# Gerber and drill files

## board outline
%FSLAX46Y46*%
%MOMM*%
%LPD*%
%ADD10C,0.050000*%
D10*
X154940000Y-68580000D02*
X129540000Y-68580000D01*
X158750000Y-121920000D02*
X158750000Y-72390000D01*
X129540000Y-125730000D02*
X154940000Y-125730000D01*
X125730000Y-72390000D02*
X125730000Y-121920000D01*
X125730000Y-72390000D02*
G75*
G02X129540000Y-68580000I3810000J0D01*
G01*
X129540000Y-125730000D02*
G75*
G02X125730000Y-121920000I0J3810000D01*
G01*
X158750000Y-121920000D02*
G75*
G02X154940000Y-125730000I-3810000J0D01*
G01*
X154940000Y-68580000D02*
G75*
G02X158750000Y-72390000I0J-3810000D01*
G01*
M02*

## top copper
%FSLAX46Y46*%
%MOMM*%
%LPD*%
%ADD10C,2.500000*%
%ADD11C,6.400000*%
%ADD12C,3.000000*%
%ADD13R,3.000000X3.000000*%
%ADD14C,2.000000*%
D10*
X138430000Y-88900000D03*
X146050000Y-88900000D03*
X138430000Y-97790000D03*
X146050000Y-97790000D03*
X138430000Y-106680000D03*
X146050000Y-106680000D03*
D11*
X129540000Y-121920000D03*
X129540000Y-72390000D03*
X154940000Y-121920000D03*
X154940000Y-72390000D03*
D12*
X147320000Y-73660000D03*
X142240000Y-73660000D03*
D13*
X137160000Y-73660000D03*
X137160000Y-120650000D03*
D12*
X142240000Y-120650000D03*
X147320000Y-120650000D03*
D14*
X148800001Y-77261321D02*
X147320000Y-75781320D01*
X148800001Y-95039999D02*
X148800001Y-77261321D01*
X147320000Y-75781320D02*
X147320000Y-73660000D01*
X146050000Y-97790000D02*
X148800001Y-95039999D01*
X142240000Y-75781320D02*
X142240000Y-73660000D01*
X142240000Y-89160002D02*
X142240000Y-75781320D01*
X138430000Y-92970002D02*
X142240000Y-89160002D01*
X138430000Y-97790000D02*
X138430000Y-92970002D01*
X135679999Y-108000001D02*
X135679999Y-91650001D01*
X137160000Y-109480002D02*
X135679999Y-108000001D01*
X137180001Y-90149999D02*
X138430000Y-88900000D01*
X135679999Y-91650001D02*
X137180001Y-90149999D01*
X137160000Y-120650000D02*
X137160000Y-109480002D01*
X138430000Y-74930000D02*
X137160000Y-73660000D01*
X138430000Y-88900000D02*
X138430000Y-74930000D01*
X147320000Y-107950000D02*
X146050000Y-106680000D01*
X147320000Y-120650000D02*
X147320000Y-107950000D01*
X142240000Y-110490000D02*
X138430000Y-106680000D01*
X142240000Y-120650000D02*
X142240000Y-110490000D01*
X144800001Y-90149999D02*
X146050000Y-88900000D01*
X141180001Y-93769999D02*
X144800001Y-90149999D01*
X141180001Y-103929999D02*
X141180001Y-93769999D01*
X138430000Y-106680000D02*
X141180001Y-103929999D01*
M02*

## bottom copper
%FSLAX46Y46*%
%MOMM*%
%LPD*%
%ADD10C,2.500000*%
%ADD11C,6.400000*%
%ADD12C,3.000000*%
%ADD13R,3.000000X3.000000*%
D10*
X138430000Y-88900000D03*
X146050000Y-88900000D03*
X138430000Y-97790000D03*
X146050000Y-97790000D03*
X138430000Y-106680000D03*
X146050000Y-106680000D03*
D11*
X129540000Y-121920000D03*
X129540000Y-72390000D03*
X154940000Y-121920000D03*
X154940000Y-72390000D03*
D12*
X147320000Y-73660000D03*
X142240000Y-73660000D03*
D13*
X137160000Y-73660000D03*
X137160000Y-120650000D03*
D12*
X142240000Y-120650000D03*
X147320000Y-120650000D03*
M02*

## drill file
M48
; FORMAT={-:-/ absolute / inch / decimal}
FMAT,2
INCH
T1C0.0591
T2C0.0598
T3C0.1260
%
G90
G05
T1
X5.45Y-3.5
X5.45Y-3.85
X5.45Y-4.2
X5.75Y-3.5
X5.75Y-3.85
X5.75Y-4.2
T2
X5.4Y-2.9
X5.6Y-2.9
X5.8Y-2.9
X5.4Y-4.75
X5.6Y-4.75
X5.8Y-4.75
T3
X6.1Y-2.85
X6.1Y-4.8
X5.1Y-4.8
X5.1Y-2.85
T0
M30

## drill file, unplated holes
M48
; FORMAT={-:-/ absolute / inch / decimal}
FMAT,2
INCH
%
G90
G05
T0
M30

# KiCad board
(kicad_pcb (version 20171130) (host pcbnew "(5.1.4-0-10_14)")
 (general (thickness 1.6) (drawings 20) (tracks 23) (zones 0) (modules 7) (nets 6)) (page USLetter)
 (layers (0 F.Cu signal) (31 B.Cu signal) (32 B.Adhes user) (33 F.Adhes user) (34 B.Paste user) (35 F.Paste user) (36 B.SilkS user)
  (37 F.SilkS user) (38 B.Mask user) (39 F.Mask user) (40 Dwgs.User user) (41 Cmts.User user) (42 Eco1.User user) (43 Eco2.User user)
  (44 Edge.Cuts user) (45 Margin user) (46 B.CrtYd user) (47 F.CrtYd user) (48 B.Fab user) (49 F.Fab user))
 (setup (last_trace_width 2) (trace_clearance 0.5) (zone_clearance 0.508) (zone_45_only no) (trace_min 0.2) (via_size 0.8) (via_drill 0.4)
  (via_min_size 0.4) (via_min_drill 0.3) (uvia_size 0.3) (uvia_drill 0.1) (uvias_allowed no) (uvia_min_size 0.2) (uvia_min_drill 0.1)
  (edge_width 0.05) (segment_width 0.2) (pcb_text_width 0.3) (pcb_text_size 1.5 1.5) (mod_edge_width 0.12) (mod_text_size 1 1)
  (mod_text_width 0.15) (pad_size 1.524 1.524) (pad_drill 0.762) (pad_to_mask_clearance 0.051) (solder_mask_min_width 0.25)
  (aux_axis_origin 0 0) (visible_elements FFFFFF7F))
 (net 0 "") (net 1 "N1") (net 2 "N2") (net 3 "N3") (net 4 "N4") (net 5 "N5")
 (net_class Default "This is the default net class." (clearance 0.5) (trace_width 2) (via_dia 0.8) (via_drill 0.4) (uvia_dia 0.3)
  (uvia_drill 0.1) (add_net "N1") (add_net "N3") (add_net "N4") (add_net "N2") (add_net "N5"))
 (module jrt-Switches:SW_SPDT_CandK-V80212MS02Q (layer F.Cu) (at 142.24 97.79)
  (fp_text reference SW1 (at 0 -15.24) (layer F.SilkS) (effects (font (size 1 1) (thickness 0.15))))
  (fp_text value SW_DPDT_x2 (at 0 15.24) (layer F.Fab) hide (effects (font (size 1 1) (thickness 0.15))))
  (pad 1 thru_hole circle (at -3.81 -8.89) (size 2.5 2.5) (drill 1.5) (layers *.Cu *.Mask) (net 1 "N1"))
  (pad 4 thru_hole circle (at 3.81 -8.89) (size 2.5 2.5) (drill 1.5) (layers *.Cu *.Mask) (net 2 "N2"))
  (pad 2 thru_hole circle (at -3.81 0) (size 2.5 2.5) (drill 1.5) (layers *.Cu *.Mask) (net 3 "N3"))
  (pad 5 thru_hole circle (at 3.81 0) (size 2.5 2.5) (drill 1.5) (layers *.Cu *.Mask) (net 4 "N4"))
  (pad 3 thru_hole circle (at -3.81 8.89) (size 2.5 2.5) (drill 1.5) (layers *.Cu *.Mask) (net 2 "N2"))
  (pad 6 thru_hole circle (at 3.81 8.89) (size 2.5 2.5) (drill 1.5) (layers *.Cu *.Mask) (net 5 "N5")))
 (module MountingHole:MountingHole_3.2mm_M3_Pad (layer F.Cu) (at 129.54 121.92)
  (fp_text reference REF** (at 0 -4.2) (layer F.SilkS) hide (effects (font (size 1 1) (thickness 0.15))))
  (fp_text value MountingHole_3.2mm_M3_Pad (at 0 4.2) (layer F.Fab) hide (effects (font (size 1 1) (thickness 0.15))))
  (pad 1 thru_hole circle (at 0 0) (size 6.4 6.4) (drill 3.2) (layers *.Cu *.Mask)))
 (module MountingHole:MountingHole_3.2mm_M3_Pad (layer F.Cu) (at 129.54 72.39)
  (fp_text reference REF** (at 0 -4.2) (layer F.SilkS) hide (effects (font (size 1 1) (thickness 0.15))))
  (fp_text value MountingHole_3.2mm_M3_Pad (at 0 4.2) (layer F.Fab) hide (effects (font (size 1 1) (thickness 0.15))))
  (pad 1 thru_hole circle (at 0 0) (size 6.4 6.4) (drill 3.2) (layers *.Cu *.Mask)))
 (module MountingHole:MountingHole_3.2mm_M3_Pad (layer F.Cu) (at 154.94 121.92)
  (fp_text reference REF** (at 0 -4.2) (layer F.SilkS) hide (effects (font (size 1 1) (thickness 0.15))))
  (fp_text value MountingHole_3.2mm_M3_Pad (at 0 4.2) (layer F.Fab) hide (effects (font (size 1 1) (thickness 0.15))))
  (pad 1 thru_hole circle (at 0 0) (size 6.4 6.4) (drill 3.2) (layers *.Cu *.Mask)))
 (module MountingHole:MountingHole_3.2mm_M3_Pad (layer F.Cu) (at 154.94 72.39)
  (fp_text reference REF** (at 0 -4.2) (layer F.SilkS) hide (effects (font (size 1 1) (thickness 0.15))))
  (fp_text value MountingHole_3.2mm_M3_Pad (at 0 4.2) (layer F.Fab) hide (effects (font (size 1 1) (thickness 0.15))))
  (pad 1 thru_hole circle (at 0 0) (size 6.4 6.4) (drill 3.2) (layers *.Cu *.Mask)))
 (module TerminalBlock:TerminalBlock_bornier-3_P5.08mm (layer F.Cu) (at 137.16 73.66)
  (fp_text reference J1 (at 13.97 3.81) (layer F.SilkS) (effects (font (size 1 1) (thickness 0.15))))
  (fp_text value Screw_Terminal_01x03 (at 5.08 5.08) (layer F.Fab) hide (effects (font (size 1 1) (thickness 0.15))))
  (pad 3 thru_hole circle (at 10.16 0) (size 3 3) (drill 1.52) (layers *.Cu *.Mask) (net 4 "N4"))
  (pad 2 thru_hole circle (at 5.08 0) (size 3 3) (drill 1.52) (layers *.Cu *.Mask) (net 3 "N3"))
  (pad 1 thru_hole rect (at 0 0) (size 3 3) (drill 1.52) (layers *.Cu *.Mask) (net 1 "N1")))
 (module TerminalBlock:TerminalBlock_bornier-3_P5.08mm (layer F.Cu) (at 137.16 120.65)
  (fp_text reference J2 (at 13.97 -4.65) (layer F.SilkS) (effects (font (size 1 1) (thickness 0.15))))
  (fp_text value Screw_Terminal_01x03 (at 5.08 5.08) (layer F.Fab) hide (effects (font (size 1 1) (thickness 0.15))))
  (pad 1 thru_hole rect (at 0 0) (size 3 3) (drill 1.52) (layers *.Cu *.Mask) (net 1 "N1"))
  (pad 2 thru_hole circle (at 5.08 0) (size 3 3) (drill 1.52) (layers *.Cu *.Mask) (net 2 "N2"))
  (pad 3 thru_hole circle (at 10.16 0) (size 3 3) (drill 1.52) (layers *.Cu *.Mask) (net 5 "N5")))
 (gr_line (start 154.94 68.58) (end 129.54 68.58) (layer Edge.Cuts) (width 0.05))
 (gr_line (start 158.75 121.92) (end 158.75 72.39) (layer Edge.Cuts) (width 0.05))
 (gr_line (start 129.54 125.73) (end 154.94 125.73) (layer Edge.Cuts) (width 0.05))
 (gr_line (start 125.73 72.39) (end 125.73 121.92) (layer Edge.Cuts) (width 0.05))
 (gr_arc (start 129.54 72.39) (end 129.54 68.58) (angle -90) (layer Edge.Cuts) (width 0.05))
 (gr_arc (start 129.54 121.92) (end 125.73 121.92) (angle -90) (layer Edge.Cuts) (width 0.05))
 (gr_arc (start 154.94 121.92) (end 154.94 125.73) (angle -90) (layer Edge.Cuts) (width 0.05))
 (gr_arc (start 154.94 72.39) (end 158.75 72.39) (angle -90) (layer Edge.Cuts) (width 0.05))
 (segment (start 148.800001 77.261321) (end 147.32 75.78132) (width 2) (layer F.Cu) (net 4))
 (segment (start 148.800001 95.039999) (end 148.800001 77.261321) (width 2) (layer F.Cu) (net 4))
 (segment (start 147.32 75.78132) (end 147.32 73.66) (width 2) (layer F.Cu) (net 4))
 (segment (start 146.05 97.79) (end 148.800001 95.039999) (width 2) (layer F.Cu) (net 4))
 (segment (start 142.24 75.78132) (end 142.24 73.66) (width 2) (layer F.Cu) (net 3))
 (segment (start 142.24 89.160002) (end 142.24 75.78132) (width 2) (layer F.Cu) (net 3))
 (segment (start 138.43 92.970002) (end 142.24 89.160002) (width 2) (layer F.Cu) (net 3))
 (segment (start 138.43 97.79) (end 138.43 92.970002) (width 2) (layer F.Cu) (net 3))
 (segment (start 135.679999 108.000001) (end 135.679999 91.650001) (width 2) (layer F.Cu) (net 1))
 (segment (start 137.16 109.480002) (end 135.679999 108.000001) (width 2) (layer F.Cu) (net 1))
 (segment (start 137.180001 90.149999) (end 138.43 88.9) (width 2) (layer F.Cu) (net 1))
 (segment (start 135.679999 91.650001) (end 137.180001 90.149999) (width 2) (layer F.Cu) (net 1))
 (segment (start 137.16 120.65) (end 137.16 109.480002) (width 2) (layer F.Cu) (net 1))
 (segment (start 138.43 74.93) (end 137.16 73.66) (width 2) (layer F.Cu) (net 1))
 (segment (start 138.43 88.9) (end 138.43 74.93) (width 2) (layer F.Cu) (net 1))
 (segment (start 147.32 107.95) (end 146.05 106.68) (width 2) (layer F.Cu) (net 5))
 (segment (start 147.32 120.65) (end 147.32 107.95) (width 2) (layer F.Cu) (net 5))
 (segment (start 142.24 110.49) (end 138.43 106.68) (width 2) (layer F.Cu) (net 2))
 (segment (start 142.24 120.65) (end 142.24 110.49) (width 2) (layer F.Cu) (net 2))
 (segment (start 144.800001 90.149999) (end 146.05 88.9) (width 2) (layer F.Cu) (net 2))
 (segment (start 141.180001 93.769999) (end 144.800001 90.149999) (width 2) (layer F.Cu) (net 2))
 (segment (start 141.180001 103.929999) (end 141.180001 93.769999) (width 2) (layer F.Cu) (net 2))
 (segment (start 138.43 106.68) (end 141.180001 103.929999) (width 2) (layer F.Cu) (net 2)))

